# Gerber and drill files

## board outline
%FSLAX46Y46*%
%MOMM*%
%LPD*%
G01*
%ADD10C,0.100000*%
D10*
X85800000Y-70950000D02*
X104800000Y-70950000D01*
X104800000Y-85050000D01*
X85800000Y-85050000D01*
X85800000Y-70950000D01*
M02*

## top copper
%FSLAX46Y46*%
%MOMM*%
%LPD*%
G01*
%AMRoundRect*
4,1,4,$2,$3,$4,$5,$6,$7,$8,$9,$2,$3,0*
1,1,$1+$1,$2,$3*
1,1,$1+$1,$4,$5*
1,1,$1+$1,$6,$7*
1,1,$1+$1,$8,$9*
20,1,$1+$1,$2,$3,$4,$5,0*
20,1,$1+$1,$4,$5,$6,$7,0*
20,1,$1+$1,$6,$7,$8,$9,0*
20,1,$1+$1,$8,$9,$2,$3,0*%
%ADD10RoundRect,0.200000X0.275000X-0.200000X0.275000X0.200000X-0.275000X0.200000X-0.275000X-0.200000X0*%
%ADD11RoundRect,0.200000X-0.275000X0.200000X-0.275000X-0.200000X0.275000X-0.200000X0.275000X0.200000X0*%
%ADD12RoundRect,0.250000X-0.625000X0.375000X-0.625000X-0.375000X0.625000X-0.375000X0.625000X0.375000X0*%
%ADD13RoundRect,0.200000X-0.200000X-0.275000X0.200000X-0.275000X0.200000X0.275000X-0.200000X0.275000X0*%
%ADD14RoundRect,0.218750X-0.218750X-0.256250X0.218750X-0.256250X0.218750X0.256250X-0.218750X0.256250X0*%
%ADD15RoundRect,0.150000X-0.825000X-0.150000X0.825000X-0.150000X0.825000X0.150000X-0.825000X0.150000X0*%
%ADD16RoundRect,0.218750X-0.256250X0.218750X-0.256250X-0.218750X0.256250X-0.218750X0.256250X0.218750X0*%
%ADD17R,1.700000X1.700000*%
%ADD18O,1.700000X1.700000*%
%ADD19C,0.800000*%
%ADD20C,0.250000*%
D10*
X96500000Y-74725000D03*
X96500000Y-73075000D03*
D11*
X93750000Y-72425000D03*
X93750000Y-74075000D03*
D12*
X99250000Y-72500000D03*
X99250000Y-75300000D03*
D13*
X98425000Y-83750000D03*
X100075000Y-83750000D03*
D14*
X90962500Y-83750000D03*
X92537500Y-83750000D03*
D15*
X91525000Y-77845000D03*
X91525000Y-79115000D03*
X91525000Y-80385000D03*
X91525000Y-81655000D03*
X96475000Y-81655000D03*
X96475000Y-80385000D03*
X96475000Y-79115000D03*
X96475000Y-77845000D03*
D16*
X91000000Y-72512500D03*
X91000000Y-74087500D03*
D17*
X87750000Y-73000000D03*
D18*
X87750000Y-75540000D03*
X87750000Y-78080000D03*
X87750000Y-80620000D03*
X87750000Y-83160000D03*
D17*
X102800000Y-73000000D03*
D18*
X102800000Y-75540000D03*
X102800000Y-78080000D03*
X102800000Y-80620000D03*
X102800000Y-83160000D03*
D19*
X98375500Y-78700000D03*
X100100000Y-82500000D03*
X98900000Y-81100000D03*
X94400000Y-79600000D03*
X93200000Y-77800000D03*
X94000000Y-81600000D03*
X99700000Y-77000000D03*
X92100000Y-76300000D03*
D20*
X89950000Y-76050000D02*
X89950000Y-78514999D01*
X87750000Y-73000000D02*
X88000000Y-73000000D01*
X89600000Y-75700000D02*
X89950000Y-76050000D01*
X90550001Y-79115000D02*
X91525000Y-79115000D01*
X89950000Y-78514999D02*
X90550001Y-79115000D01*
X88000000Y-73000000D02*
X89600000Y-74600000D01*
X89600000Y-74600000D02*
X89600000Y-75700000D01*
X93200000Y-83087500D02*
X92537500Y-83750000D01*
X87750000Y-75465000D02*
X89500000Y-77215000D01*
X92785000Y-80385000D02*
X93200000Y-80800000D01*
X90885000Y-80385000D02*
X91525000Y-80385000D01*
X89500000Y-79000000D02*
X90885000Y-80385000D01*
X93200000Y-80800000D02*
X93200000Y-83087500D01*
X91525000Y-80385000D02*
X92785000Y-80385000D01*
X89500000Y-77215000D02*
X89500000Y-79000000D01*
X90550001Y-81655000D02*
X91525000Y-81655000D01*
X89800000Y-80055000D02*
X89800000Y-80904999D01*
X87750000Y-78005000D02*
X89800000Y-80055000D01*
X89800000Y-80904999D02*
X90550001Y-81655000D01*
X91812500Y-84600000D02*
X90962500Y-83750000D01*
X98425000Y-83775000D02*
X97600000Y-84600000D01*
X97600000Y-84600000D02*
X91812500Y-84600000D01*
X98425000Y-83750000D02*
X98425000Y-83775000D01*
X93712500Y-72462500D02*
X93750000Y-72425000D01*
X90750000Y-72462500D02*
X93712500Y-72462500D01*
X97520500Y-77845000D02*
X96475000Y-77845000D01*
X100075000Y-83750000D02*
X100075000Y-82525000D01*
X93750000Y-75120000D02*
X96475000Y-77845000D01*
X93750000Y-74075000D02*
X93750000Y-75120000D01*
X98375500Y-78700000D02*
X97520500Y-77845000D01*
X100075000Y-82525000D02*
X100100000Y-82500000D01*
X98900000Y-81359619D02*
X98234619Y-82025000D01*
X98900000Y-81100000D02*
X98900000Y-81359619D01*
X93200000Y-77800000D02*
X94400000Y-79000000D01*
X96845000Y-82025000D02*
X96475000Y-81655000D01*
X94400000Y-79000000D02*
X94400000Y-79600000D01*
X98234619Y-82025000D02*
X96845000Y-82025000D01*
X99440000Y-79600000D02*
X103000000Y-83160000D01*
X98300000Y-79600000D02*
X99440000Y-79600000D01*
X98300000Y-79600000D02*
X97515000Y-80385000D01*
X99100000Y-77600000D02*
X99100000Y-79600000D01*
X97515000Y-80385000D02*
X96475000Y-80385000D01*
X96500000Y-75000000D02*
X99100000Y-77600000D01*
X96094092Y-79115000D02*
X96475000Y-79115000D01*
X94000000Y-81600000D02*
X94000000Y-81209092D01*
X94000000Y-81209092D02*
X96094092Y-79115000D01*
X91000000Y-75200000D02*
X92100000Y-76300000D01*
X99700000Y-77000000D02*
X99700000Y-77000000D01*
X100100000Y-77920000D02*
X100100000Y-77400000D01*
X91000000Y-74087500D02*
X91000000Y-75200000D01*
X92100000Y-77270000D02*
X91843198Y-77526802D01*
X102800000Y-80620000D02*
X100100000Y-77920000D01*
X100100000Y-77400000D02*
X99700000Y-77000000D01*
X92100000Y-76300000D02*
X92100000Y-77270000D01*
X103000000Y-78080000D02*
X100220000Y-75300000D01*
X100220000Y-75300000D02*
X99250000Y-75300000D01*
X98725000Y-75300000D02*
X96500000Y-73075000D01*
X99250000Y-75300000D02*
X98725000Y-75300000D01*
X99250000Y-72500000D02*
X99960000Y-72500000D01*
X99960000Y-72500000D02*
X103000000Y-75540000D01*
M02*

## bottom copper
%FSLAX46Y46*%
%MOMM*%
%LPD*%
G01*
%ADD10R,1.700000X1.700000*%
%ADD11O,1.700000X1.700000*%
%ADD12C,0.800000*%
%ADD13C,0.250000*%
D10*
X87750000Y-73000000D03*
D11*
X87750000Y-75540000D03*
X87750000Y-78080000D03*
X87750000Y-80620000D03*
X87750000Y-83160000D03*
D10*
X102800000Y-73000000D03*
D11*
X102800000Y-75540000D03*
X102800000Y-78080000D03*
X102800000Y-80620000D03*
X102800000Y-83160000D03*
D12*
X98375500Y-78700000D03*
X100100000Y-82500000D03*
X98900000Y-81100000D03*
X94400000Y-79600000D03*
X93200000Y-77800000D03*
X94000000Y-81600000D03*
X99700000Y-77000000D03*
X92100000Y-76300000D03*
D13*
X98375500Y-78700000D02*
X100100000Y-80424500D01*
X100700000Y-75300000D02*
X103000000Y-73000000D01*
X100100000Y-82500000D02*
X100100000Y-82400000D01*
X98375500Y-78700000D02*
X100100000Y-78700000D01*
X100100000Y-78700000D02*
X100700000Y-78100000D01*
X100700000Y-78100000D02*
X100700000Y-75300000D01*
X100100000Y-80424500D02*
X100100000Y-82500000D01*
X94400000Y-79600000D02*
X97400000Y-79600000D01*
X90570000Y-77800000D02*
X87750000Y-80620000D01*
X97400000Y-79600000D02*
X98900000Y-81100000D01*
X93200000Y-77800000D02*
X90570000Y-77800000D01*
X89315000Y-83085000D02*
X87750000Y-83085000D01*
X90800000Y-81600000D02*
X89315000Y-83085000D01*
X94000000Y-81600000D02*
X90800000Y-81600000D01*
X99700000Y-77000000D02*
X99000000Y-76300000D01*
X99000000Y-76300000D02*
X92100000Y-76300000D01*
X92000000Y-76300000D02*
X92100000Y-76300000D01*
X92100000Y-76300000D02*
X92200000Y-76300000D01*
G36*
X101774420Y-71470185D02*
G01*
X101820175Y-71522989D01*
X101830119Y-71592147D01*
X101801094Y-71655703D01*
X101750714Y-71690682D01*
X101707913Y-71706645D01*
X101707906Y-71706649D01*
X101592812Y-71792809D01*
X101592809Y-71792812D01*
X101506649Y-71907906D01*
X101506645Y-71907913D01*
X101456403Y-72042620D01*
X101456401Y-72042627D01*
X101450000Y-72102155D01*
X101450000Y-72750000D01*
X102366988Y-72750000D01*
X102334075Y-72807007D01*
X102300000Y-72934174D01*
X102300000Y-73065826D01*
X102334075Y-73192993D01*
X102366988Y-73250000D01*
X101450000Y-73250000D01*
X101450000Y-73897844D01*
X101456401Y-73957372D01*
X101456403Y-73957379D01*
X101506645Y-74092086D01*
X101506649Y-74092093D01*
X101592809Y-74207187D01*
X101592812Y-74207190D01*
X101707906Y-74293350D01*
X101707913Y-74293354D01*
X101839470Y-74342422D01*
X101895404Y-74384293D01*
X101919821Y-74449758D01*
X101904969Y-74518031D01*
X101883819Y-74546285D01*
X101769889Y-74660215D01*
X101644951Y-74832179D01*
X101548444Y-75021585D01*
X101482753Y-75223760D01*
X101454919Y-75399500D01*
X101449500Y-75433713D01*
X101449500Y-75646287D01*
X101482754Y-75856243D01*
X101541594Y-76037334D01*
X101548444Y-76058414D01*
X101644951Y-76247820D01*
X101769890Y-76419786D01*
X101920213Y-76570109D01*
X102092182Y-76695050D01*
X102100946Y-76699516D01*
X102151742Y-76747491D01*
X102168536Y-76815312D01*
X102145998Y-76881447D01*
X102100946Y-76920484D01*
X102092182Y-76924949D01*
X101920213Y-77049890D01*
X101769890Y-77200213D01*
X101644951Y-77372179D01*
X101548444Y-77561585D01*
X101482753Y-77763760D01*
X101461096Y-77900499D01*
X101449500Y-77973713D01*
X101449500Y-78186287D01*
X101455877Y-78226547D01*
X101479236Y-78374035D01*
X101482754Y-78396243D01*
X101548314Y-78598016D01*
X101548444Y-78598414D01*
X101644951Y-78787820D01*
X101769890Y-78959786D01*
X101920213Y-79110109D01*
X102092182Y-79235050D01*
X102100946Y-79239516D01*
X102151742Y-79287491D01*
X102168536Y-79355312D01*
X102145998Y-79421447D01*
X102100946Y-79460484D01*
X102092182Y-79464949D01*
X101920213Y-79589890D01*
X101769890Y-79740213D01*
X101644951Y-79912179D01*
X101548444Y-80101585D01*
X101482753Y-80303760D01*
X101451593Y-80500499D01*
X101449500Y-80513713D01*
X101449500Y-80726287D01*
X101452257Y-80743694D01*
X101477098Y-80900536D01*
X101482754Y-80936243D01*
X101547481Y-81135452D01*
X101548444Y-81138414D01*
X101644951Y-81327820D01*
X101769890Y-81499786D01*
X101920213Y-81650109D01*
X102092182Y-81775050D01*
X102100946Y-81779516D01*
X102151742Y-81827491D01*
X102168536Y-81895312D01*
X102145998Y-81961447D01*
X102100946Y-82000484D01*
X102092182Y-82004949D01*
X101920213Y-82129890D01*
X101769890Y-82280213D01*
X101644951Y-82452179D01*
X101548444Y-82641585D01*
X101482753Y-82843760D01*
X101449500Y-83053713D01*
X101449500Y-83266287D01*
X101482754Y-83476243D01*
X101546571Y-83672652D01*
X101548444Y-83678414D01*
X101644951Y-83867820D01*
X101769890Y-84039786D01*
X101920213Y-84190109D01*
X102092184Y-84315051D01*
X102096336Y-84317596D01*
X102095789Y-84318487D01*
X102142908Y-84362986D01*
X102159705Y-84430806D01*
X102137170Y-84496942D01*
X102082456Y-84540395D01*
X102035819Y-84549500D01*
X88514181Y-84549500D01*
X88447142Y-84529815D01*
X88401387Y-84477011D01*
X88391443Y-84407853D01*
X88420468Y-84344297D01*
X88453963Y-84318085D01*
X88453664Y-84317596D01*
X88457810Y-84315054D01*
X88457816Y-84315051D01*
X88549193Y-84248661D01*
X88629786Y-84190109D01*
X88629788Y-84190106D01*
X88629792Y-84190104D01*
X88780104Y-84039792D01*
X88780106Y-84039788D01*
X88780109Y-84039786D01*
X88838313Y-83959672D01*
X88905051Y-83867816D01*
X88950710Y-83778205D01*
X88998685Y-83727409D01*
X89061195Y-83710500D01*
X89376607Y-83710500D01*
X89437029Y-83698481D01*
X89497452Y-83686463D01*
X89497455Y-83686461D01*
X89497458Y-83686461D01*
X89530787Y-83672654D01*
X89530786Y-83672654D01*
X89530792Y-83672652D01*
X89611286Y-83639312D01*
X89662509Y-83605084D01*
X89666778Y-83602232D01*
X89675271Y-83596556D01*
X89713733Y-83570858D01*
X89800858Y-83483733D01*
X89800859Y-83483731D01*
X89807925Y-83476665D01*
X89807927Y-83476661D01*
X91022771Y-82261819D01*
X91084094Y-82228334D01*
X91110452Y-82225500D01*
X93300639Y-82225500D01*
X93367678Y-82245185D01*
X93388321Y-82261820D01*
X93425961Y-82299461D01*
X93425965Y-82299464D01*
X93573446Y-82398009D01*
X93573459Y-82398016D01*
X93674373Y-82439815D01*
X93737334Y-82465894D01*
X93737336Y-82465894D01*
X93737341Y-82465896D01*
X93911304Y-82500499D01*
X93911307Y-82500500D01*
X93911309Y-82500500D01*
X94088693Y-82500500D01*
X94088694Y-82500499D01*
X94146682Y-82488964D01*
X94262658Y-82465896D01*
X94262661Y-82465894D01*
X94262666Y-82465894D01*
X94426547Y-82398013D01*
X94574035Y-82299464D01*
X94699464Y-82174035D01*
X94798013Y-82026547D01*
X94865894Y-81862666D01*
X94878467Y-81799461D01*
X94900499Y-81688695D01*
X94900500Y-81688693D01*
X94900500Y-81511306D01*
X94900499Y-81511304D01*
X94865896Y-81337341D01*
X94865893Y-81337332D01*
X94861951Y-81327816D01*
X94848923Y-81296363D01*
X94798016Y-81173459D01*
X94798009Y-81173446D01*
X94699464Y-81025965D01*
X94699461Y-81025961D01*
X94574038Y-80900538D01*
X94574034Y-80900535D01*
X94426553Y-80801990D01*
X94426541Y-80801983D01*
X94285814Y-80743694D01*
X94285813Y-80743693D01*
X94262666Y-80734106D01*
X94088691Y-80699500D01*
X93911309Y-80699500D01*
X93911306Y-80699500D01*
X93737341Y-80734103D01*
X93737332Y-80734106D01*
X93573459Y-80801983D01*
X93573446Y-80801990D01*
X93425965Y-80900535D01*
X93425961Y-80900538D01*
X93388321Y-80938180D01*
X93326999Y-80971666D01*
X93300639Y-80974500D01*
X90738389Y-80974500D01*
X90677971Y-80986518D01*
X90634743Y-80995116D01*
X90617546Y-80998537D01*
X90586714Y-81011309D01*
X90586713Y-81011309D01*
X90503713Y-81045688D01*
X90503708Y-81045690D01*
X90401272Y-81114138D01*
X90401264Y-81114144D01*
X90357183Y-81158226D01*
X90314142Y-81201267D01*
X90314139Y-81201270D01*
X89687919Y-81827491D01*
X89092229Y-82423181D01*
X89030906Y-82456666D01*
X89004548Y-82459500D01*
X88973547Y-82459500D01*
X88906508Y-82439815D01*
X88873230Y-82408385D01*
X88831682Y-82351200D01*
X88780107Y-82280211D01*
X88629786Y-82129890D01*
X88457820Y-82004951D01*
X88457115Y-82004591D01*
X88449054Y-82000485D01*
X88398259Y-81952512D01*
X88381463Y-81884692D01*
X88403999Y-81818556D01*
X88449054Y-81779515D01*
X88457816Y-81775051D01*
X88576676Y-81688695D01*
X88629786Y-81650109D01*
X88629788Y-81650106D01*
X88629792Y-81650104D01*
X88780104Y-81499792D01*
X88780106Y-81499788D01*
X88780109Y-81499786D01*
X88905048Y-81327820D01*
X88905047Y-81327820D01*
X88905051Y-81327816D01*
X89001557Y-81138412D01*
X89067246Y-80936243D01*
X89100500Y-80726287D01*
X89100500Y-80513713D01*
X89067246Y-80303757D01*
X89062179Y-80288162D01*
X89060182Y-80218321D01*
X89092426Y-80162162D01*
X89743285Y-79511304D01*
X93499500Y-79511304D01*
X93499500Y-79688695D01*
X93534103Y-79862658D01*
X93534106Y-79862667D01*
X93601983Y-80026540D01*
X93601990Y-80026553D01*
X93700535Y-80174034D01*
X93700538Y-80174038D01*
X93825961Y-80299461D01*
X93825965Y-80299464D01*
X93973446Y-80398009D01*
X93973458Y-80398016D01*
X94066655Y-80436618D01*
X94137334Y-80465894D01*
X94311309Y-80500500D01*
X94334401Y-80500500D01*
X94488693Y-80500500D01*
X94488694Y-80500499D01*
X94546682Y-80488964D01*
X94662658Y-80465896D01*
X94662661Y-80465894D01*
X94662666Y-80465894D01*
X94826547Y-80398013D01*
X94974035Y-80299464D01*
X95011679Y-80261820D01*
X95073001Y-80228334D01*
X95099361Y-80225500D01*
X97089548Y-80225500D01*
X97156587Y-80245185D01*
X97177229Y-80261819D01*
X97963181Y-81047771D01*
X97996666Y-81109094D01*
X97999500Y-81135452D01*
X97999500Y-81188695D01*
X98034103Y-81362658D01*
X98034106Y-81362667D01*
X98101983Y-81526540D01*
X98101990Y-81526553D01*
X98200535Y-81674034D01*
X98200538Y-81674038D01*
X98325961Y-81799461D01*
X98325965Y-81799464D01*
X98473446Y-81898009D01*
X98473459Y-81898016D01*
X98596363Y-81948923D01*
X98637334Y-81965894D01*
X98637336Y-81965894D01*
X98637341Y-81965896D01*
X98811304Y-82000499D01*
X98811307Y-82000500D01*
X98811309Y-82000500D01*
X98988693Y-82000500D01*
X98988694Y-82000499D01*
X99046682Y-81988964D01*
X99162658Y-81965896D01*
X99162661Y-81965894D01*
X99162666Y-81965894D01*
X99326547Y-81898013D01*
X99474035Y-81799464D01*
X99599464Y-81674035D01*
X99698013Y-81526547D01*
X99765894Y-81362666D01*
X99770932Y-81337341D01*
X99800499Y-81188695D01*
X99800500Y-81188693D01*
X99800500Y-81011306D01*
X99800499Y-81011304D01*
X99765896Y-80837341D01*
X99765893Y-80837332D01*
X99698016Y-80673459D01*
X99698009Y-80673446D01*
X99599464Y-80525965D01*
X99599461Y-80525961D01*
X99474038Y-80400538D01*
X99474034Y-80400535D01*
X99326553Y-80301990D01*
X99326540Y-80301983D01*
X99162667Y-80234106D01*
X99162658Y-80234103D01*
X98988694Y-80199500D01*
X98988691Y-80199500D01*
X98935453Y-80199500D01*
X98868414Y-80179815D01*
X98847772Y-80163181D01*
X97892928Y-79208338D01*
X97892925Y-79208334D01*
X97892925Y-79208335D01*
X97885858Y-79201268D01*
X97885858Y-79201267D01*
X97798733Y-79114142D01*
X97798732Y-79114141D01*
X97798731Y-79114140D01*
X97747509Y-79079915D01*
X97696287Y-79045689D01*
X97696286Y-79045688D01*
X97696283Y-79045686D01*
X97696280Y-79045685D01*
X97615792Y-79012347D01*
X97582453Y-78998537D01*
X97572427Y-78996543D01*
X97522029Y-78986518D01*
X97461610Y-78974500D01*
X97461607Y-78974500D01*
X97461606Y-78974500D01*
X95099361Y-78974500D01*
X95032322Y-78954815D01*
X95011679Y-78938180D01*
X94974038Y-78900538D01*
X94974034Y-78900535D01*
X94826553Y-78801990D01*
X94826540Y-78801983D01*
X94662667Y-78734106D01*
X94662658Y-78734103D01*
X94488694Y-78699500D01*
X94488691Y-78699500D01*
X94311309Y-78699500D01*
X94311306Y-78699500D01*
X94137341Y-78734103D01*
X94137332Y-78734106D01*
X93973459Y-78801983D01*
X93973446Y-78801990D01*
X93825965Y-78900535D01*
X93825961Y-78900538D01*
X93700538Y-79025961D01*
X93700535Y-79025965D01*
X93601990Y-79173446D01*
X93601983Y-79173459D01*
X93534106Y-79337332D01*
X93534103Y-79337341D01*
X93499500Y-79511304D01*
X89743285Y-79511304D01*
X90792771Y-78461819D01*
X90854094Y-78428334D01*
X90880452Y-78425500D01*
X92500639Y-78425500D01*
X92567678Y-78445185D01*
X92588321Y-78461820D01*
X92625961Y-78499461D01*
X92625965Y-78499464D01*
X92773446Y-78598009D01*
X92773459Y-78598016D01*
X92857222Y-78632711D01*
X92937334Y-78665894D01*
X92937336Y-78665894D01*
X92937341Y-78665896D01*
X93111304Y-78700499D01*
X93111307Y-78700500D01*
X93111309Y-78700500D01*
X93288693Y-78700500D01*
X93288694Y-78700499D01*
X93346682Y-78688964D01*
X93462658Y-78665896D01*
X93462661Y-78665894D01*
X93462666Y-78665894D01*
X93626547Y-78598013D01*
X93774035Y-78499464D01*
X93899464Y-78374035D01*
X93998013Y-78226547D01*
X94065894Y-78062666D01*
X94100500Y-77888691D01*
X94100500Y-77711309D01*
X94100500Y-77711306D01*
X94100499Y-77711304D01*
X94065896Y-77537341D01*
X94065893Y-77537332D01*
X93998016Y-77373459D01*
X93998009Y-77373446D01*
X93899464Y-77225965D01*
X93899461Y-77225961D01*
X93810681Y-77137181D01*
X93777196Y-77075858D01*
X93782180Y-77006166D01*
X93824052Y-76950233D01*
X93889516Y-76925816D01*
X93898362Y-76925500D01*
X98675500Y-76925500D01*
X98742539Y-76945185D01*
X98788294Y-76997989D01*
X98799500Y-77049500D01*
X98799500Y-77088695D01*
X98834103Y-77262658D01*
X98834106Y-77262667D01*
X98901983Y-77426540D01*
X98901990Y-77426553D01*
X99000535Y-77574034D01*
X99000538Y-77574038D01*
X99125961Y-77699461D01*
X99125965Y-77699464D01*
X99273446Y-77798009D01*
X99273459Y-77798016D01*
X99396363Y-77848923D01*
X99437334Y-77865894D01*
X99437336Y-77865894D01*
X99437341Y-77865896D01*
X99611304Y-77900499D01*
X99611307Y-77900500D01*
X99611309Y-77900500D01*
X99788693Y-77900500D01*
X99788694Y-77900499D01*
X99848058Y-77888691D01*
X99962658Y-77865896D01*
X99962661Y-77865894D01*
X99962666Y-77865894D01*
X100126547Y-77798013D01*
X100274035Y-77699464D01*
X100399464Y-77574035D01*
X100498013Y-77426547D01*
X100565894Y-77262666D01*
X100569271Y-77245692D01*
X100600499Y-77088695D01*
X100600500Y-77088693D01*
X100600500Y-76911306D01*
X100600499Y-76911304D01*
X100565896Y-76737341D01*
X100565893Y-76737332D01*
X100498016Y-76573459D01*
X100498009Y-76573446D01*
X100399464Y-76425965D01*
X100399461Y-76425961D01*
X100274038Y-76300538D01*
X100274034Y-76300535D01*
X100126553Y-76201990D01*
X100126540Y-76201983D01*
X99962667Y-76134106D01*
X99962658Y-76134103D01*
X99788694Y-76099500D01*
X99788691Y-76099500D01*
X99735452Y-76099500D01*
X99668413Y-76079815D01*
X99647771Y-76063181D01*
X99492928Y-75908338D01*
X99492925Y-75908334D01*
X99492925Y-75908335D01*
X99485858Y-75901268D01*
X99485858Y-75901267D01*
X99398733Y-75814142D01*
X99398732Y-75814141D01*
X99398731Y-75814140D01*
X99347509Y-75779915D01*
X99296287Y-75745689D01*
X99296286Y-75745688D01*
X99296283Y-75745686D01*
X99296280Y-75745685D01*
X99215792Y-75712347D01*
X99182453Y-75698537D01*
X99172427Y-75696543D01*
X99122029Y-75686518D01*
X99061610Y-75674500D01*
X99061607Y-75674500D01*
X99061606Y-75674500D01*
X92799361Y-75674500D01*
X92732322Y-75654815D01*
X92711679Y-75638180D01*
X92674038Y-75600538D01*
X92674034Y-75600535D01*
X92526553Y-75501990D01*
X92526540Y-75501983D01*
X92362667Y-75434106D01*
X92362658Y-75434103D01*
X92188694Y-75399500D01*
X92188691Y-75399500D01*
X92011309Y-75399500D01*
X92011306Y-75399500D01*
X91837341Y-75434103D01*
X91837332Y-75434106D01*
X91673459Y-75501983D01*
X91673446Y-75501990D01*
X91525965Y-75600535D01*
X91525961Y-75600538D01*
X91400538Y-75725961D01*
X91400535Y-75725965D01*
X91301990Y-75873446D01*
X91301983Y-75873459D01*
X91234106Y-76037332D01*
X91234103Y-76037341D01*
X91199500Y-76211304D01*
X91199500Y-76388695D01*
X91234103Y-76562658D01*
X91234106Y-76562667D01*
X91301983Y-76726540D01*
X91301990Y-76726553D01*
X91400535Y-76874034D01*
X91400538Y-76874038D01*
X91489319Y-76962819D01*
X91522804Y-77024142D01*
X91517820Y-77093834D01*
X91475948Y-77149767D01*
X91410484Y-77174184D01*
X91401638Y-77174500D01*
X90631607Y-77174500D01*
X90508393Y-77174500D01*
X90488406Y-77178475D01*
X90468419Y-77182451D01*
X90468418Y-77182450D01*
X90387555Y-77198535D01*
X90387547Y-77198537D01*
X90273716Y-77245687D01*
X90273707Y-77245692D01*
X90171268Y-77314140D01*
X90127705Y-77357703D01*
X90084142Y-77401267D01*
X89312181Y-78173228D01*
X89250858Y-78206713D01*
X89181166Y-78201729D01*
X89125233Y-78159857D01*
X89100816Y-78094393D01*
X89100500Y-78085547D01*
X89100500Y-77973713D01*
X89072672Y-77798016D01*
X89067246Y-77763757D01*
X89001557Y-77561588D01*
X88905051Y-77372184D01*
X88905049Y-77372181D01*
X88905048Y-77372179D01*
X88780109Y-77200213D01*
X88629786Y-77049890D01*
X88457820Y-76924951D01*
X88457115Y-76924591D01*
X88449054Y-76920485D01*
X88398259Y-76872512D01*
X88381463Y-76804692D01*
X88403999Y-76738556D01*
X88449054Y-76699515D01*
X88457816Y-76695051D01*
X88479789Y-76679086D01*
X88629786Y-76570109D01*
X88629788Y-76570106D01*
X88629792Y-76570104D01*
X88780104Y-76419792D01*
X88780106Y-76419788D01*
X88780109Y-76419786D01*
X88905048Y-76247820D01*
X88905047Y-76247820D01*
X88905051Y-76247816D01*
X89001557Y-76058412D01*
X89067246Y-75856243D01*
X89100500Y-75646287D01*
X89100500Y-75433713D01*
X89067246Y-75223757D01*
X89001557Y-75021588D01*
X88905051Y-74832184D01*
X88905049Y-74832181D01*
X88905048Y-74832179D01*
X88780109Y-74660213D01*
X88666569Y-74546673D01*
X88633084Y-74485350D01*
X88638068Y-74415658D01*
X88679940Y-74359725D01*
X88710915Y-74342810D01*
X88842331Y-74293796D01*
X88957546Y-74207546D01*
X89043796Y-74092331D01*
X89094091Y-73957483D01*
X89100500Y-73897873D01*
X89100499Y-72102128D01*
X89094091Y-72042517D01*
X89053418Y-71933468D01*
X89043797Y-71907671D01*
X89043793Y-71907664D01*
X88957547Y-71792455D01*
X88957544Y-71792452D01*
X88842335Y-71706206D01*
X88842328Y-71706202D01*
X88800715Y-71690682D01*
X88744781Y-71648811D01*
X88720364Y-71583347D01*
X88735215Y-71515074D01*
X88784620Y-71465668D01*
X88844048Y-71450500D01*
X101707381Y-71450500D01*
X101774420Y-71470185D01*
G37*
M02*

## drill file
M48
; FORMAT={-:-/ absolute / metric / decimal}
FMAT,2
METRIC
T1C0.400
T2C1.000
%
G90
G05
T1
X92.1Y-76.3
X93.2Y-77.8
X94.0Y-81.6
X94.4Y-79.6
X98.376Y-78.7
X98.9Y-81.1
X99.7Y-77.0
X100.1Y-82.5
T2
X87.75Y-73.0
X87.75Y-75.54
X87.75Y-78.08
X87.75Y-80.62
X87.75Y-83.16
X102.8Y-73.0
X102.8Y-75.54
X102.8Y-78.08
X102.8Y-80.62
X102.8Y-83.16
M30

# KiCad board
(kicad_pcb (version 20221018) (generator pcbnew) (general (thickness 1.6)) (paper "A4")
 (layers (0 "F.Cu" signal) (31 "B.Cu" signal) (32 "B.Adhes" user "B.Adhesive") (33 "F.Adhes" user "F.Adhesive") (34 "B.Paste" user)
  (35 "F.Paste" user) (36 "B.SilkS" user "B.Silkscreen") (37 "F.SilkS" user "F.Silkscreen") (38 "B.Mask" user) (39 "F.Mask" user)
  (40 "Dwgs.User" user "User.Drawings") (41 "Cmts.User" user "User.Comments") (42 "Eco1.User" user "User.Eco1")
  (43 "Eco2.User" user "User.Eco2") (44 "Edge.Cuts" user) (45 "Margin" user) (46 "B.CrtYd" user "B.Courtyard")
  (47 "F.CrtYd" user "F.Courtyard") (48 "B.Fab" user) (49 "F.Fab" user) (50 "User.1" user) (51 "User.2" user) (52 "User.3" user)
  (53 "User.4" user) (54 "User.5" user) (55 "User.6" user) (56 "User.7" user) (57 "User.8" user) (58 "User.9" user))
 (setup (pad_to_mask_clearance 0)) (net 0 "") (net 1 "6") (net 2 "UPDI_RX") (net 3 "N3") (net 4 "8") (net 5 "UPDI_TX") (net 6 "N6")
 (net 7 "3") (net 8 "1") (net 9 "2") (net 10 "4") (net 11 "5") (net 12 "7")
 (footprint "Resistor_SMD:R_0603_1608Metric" (layer "F.Cu") (at 96.5 73.9 90)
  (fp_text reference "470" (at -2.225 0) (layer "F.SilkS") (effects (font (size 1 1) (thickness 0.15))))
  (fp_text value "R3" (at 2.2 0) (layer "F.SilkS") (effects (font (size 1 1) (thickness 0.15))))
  (pad "1" smd roundrect (at -0.825 0 90) (size 0.8 0.95) (layers "F.Cu" "F.Paste" "F.Mask") (roundrect_rratio 0.25) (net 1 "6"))
  (pad "2" smd roundrect (at 0.825 0 90) (size 0.8 0.95) (layers "F.Cu" "F.Paste" "F.Mask") (roundrect_rratio 0.25) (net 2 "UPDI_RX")))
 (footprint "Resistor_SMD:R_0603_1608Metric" (layer "F.Cu") (at 93.75 73.25 -90)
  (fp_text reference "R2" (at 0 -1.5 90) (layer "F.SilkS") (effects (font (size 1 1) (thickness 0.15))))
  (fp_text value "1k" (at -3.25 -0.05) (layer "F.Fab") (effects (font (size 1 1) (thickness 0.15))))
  (pad "1" smd roundrect (at -0.825 0 270) (size 0.8 0.95) (layers "F.Cu" "F.Paste" "F.Mask") (roundrect_rratio 0.25) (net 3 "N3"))
  (pad "2" smd roundrect (at 0.825 0 270) (size 0.8 0.95) (layers "F.Cu" "F.Paste" "F.Mask") (roundrect_rratio 0.25) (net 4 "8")))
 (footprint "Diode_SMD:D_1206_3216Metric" (layer "F.Cu") (at 99.25 73.9 -90)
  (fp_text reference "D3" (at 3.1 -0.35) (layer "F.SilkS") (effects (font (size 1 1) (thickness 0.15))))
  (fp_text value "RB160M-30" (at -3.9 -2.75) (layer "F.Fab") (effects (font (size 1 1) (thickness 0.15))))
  (pad "1" smd roundrect (at -1.4 0 270) (size 1.25 1.75) (layers "F.Cu" "F.Paste" "F.Mask") (roundrect_rratio 0.2) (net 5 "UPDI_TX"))
  (pad "2" smd roundrect (at 1.4 0 270) (size 1.25 1.75) (layers "F.Cu" "F.Paste" "F.Mask") (roundrect_rratio 0.2) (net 2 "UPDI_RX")))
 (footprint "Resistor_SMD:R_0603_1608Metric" (layer "F.Cu") (at 99.25 83.75)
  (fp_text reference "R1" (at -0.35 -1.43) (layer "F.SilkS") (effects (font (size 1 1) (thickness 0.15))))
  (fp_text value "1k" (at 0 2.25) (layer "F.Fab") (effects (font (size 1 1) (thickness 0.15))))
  (pad "1" smd roundrect (at -0.825 0) (size 0.8 0.95) (layers "F.Cu" "F.Paste" "F.Mask") (roundrect_rratio 0.25) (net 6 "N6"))
  (pad "2" smd roundrect (at 0.825 0) (size 0.8 0.95) (layers "F.Cu" "F.Paste" "F.Mask") (roundrect_rratio 0.25) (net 4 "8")))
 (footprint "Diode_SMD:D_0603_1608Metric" (layer "F.Cu") (at 91.75 83.75)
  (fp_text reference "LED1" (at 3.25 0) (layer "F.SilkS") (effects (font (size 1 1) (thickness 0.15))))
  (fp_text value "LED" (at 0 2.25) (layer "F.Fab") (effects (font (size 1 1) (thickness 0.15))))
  (pad "1" smd roundrect (at -0.7875 0) (size 0.875 0.95) (layers "F.Cu" "F.Paste" "F.Mask") (roundrect_rratio 0.25) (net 6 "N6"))
  (pad "2" smd roundrect (at 0.7875 0) (size 0.875 0.95) (layers "F.Cu" "F.Paste" "F.Mask") (roundrect_rratio 0.25) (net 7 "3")))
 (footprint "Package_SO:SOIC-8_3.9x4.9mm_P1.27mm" (layer "F.Cu") (at 94 79.75)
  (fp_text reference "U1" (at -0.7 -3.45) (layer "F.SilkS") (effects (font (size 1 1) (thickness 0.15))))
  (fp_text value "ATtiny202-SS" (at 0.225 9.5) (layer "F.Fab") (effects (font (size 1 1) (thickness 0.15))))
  (pad "1" smd roundrect (at -2.475 -1.905) (size 1.95 0.6) (layers "F.Cu" "F.Paste" "F.Mask") (roundrect_rratio 0.25) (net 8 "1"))
  (pad "2" smd roundrect (at -2.475 -0.635) (size 1.95 0.6) (layers "F.Cu" "F.Paste" "F.Mask") (roundrect_rratio 0.25) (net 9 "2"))
  (pad "3" smd roundrect (at -2.475 0.635) (size 1.95 0.6) (layers "F.Cu" "F.Paste" "F.Mask") (roundrect_rratio 0.25) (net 7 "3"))
  (pad "4" smd roundrect (at -2.475 1.905) (size 1.95 0.6) (layers "F.Cu" "F.Paste" "F.Mask") (roundrect_rratio 0.25) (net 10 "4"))
  (pad "5" smd roundrect (at 2.475 1.905) (size 1.95 0.6) (layers "F.Cu" "F.Paste" "F.Mask") (roundrect_rratio 0.25) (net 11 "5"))
  (pad "6" smd roundrect (at 2.475 0.635) (size 1.95 0.6) (layers "F.Cu" "F.Paste" "F.Mask") (roundrect_rratio 0.25) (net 1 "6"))
  (pad "7" smd roundrect (at 2.475 -0.635) (size 1.95 0.6) (layers "F.Cu" "F.Paste" "F.Mask") (roundrect_rratio 0.25) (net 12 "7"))
  (pad "8" smd roundrect (at 2.475 -1.905) (size 1.95 0.6) (layers "F.Cu" "F.Paste" "F.Mask") (roundrect_rratio 0.25) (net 4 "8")))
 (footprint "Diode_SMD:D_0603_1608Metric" (layer "F.Cu") (at 91 73.3 -90)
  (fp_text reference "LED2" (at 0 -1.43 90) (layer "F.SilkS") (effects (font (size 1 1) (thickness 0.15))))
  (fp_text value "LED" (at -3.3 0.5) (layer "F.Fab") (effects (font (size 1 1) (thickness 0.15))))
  (pad "1" smd roundrect (at -0.7875 0 270) (size 0.875 0.95) (layers "F.Cu" "F.Paste" "F.Mask") (roundrect_rratio 0.25) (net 3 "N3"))
  (pad "2" smd roundrect (at 0.7875 0 270) (size 0.875 0.95) (layers "F.Cu" "F.Paste" "F.Mask") (roundrect_rratio 0.25) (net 8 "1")))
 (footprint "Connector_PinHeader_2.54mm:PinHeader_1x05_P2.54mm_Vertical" (layer "B.Cu") (at 87.75 73 180)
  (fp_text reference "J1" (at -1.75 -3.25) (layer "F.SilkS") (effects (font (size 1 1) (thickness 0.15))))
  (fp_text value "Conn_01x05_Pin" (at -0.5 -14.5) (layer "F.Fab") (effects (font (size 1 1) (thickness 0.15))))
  (pad "1" thru_hole rect (at 0 0 180) (size 1.7 1.7) (drill 1) (layers "*.Cu" "*.Mask") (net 9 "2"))
  (pad "2" thru_hole oval (at 0 -2.54 180) (size 1.7 1.7) (drill 1) (layers "*.Cu" "*.Mask") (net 7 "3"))
  (pad "3" thru_hole oval (at 0 -5.08 180) (size 1.7 1.7) (drill 1) (layers "*.Cu" "*.Mask") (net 10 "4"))
  (pad "4" thru_hole oval (at 0 -7.62 180) (size 1.7 1.7) (drill 1) (layers "*.Cu" "*.Mask") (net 11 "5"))
  (pad "5" thru_hole oval (at 0 -10.16 180) (size 1.7 1.7) (drill 1) (layers "*.Cu" "*.Mask") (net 12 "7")))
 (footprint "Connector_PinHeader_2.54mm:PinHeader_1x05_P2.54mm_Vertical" (layer "B.Cu") (at 102.8 73 180)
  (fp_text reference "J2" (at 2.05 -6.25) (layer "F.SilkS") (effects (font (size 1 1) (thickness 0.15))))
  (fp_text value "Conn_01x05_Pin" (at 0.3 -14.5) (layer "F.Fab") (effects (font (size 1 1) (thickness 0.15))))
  (pad "1" thru_hole rect (at 0 0 180) (size 1.7 1.7) (drill 1) (layers "*.Cu" "*.Mask") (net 4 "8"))
  (pad "2" thru_hole oval (at 0 -2.54 180) (size 1.7 1.7) (drill 1) (layers "*.Cu" "*.Mask") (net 5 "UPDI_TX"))
  (pad "3" thru_hole oval (at 0 -5.08 180) (size 1.7 1.7) (drill 1) (layers "*.Cu" "*.Mask") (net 2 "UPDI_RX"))
  (pad "4" thru_hole oval (at 0 -7.62 180) (size 1.7 1.7) (drill 1) (layers "*.Cu" "*.Mask") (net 8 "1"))
  (pad "5" thru_hole oval (at 0 -10.16 180) (size 1.7 1.7) (drill 1) (layers "*.Cu" "*.Mask") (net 1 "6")))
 (gr_rect (start 85.8 70.95) (end 104.8 85.05) (stroke (width 0.1) (type default)) (fill none) (layer "Edge.Cuts"))
 (segment (start 89.95 76.05) (end 89.95 78.514999) (width 0.25) (layer "F.Cu") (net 9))
 (segment (start 87.75 73) (end 88 73) (width 0.25) (layer "F.Cu") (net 9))
 (segment (start 89.6 75.7) (end 89.95 76.05) (width 0.25) (layer "F.Cu") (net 9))
 (segment (start 90.550001 79.115) (end 91.525 79.115) (width 0.25) (layer "F.Cu") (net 9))
 (segment (start 89.95 78.514999) (end 90.550001 79.115) (width 0.25) (layer "F.Cu") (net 9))
 (segment (start 88 73) (end 89.6 74.6) (width 0.25) (layer "F.Cu") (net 9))
 (segment (start 89.6 74.6) (end 89.6 75.7) (width 0.25) (layer "F.Cu") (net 9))
 (segment (start 93.2 83.0875) (end 92.5375 83.75) (width 0.25) (layer "F.Cu") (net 7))
 (segment (start 87.75 75.465) (end 89.5 77.215) (width 0.25) (layer "F.Cu") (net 7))
 (segment (start 92.785 80.385) (end 93.2 80.8) (width 0.25) (layer "F.Cu") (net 7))
 (segment (start 90.885 80.385) (end 91.525 80.385) (width 0.25) (layer "F.Cu") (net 7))
 (segment (start 89.5 79) (end 90.885 80.385) (width 0.25) (layer "F.Cu") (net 7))
 (segment (start 93.2 80.8) (end 93.2 83.0875) (width 0.25) (layer "F.Cu") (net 7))
 (segment (start 91.525 80.385) (end 92.785 80.385) (width 0.25) (layer "F.Cu") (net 7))
 (segment (start 89.5 77.215) (end 89.5 79) (width 0.25) (layer "F.Cu") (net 7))
 (segment (start 90.550001 81.655) (end 91.525 81.655) (width 0.25) (layer "F.Cu") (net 10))
 (segment (start 89.8 80.055) (end 89.8 80.904999) (width 0.25) (layer "F.Cu") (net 10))
 (segment (start 87.75 78.005) (end 89.8 80.055) (width 0.25) (layer "F.Cu") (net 10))
 (segment (start 89.8 80.904999) (end 90.550001 81.655) (width 0.25) (layer "F.Cu") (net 10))
 (segment (start 91.8125 84.6) (end 90.9625 83.75) (width 0.25) (layer "F.Cu") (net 6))
 (segment (start 98.425 83.775) (end 97.6 84.6) (width 0.25) (layer "F.Cu") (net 6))
 (segment (start 97.6 84.6) (end 91.8125 84.6) (width 0.25) (layer "F.Cu") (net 6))
 (segment (start 98.425 83.75) (end 98.425 83.775) (width 0.25) (layer "F.Cu") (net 6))
 (segment (start 93.7125 72.4625) (end 93.75 72.425) (width 0.25) (layer "F.Cu") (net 3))
 (segment (start 90.75 72.4625) (end 93.7125 72.4625) (width 0.25) (layer "F.Cu") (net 3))
 (segment (start 97.5205 77.845) (end 96.475 77.845) (width 0.25) (layer "F.Cu") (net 4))
 (segment (start 100.075 83.75) (end 100.075 82.525) (width 0.25) (layer "F.Cu") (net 4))
 (segment (start 93.75 75.12) (end 96.475 77.845) (width 0.25) (layer "F.Cu") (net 4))
 (segment (start 93.75 74.075) (end 93.75 75.12) (width 0.25) (layer "F.Cu") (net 4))
 (segment (start 98.3755 78.7) (end 97.5205 77.845) (width 0.25) (layer "F.Cu") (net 4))
 (segment (start 100.075 82.525) (end 100.1 82.5) (width 0.25) (layer "F.Cu") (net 4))
 (via (at 98.3755 78.7) (size 0.8) (drill 0.4) (layers "F.Cu" "B.Cu") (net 4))
 (via (at 100.1 82.5) (size 0.8) (drill 0.4) (layers "F.Cu" "B.Cu") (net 4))
 (segment (start 98.3755 78.7) (end 100.1 80.4245) (width 0.25) (layer "B.Cu") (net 4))
 (segment (start 100.7 75.3) (end 103 73) (width 0.25) (layer "B.Cu") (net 4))
 (segment (start 100.1 82.5) (end 100.1 82.4) (width 0.25) (layer "B.Cu") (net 4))
 (segment (start 98.3755 78.7) (end 100.1 78.7) (width 0.25) (layer "B.Cu") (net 4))
 (segment (start 100.1 78.7) (end 100.7 78.1) (width 0.25) (layer "B.Cu") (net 4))
 (segment (start 100.7 78.1) (end 100.7 75.3) (width 0.25) (layer "B.Cu") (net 4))
 (segment (start 100.1 80.4245) (end 100.1 82.5) (width 0.25) (layer "B.Cu") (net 4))
 (segment (start 98.9 81.359619) (end 98.234619 82.025) (width 0.25) (layer "F.Cu") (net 11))
 (segment (start 98.9 81.1) (end 98.9 81.359619) (width 0.25) (layer "F.Cu") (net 11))
 (segment (start 93.2 77.8) (end 94.4 79) (width 0.25) (layer "F.Cu") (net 11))
 (segment (start 96.845 82.025) (end 96.475 81.655) (width 0.25) (layer "F.Cu") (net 11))
 (segment (start 94.4 79) (end 94.4 79.6) (width 0.25) (layer "F.Cu") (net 11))
 (segment (start 98.234619 82.025) (end 96.845 82.025) (width 0.25) (layer "F.Cu") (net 11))
 (via (at 98.9 81.1) (size 0.8) (drill 0.4) (layers "F.Cu" "B.Cu") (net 11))
 (via (at 94.4 79.6) (size 0.8) (drill 0.4) (layers "F.Cu" "B.Cu") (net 11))
 (via (at 93.2 77.8) (size 0.8) (drill 0.4) (layers "F.Cu" "B.Cu") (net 11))
 (segment (start 94.4 79.6) (end 97.4 79.6) (width 0.25) (layer "B.Cu") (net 11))
 (segment (start 90.57 77.8) (end 87.75 80.62) (width 0.25) (layer "B.Cu") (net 11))
 (segment (start 97.4 79.6) (end 98.9 81.1) (width 0.25) (layer "B.Cu") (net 11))
 (segment (start 93.2 77.8) (end 90.57 77.8) (width 0.25) (layer "B.Cu") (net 11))
 (segment (start 99.44 79.6) (end 103 83.16) (width 0.25) (layer "F.Cu") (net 1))
 (segment (start 98.3 79.6) (end 99.44 79.6) (width 0.25) (layer "F.Cu") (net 1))
 (segment (start 98.3 79.6) (end 97.515 80.385) (width 0.25) (layer "F.Cu") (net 1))
 (segment (start 99.1 77.6) (end 99.1 79.6) (width 0.25) (layer "F.Cu") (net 1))
 (segment (start 97.515 80.385) (end 96.475 80.385) (width 0.25) (layer "F.Cu") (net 1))
 (segment (start 96.5 75) (end 99.1 77.6) (width 0.25) (layer "F.Cu") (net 1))
 (segment (start 96.094092 79.115) (end 96.475 79.115) (width 0.25) (layer "F.Cu") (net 12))
 (segment (start 94 81.6) (end 94 81.209092) (width 0.25) (layer "F.Cu") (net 12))
 (segment (start 94 81.209092) (end 96.094092 79.115) (width 0.25) (layer "F.Cu") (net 12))
 (via (at 94 81.6) (size 0.8) (drill 0.4) (layers "F.Cu" "B.Cu") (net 12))
 (segment (start 89.315 83.085) (end 87.75 83.085) (width 0.25) (layer "B.Cu") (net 12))
 (segment (start 90.8 81.6) (end 89.315 83.085) (width 0.25) (layer "B.Cu") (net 12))
 (segment (start 94 81.6) (end 90.8 81.6) (width 0.25) (layer "B.Cu") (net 12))
 (segment (start 91 75.2) (end 92.1 76.3) (width 0.25) (layer "F.Cu") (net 8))
 (segment (start 99.7 77) (end 99.7 77) (width 0.25) (layer "F.Cu") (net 8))
 (segment (start 100.1 77.92) (end 100.1 77.4) (width 0.25) (layer "F.Cu") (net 8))
 (segment (start 91 74.0875) (end 91 75.2) (width 0.25) (layer "F.Cu") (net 8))
 (segment (start 92.1 77.27) (end 91.843198 77.526802) (width 0.25) (layer "F.Cu") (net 8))
 (segment (start 102.8 80.62) (end 100.1 77.92) (width 0.25) (layer "F.Cu") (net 8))
 (segment (start 100.1 77.4) (end 99.7 77) (width 0.25) (layer "F.Cu") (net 8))
 (segment (start 92.1 76.3) (end 92.1 77.27) (width 0.25) (layer "F.Cu") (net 8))
 (via (at 99.7 77) (size 0.8) (drill 0.4) (layers "F.Cu" "B.Cu") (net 8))
 (via (at 92.1 76.3) (size 0.8) (drill 0.4) (layers "F.Cu" "B.Cu") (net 8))
 (segment (start 99.7 77) (end 99 76.3) (width 0.25) (layer "B.Cu") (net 8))
 (segment (start 99 76.3) (end 92.1 76.3) (width 0.25) (layer "B.Cu") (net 8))
 (segment (start 92 76.3) (end 92.1 76.3) (width 0.25) (layer "B.Cu") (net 8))
 (segment (start 92.1 76.3) (end 92.2 76.3) (width 0.25) (layer "B.Cu") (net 8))
 (segment (start 103 78.08) (end 100.22 75.3) (width 0.25) (layer "F.Cu") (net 2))
 (segment (start 100.22 75.3) (end 99.25 75.3) (width 0.25) (layer "F.Cu") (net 2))
 (segment (start 98.725 75.3) (end 96.5 73.075) (width 0.25) (layer "F.Cu") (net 2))
 (segment (start 99.25 75.3) (end 98.725 75.3) (width 0.25) (layer "F.Cu") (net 2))
 (segment (start 99.25 72.5) (end 99.96 72.5) (width 0.25) (layer "F.Cu") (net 5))
 (segment (start 99.96 72.5) (end 103 75.54) (width 0.25) (layer "F.Cu") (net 5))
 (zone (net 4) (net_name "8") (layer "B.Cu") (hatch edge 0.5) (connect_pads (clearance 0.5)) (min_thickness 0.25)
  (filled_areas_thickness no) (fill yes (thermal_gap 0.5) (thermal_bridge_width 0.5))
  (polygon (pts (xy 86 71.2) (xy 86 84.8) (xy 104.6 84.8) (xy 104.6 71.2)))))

